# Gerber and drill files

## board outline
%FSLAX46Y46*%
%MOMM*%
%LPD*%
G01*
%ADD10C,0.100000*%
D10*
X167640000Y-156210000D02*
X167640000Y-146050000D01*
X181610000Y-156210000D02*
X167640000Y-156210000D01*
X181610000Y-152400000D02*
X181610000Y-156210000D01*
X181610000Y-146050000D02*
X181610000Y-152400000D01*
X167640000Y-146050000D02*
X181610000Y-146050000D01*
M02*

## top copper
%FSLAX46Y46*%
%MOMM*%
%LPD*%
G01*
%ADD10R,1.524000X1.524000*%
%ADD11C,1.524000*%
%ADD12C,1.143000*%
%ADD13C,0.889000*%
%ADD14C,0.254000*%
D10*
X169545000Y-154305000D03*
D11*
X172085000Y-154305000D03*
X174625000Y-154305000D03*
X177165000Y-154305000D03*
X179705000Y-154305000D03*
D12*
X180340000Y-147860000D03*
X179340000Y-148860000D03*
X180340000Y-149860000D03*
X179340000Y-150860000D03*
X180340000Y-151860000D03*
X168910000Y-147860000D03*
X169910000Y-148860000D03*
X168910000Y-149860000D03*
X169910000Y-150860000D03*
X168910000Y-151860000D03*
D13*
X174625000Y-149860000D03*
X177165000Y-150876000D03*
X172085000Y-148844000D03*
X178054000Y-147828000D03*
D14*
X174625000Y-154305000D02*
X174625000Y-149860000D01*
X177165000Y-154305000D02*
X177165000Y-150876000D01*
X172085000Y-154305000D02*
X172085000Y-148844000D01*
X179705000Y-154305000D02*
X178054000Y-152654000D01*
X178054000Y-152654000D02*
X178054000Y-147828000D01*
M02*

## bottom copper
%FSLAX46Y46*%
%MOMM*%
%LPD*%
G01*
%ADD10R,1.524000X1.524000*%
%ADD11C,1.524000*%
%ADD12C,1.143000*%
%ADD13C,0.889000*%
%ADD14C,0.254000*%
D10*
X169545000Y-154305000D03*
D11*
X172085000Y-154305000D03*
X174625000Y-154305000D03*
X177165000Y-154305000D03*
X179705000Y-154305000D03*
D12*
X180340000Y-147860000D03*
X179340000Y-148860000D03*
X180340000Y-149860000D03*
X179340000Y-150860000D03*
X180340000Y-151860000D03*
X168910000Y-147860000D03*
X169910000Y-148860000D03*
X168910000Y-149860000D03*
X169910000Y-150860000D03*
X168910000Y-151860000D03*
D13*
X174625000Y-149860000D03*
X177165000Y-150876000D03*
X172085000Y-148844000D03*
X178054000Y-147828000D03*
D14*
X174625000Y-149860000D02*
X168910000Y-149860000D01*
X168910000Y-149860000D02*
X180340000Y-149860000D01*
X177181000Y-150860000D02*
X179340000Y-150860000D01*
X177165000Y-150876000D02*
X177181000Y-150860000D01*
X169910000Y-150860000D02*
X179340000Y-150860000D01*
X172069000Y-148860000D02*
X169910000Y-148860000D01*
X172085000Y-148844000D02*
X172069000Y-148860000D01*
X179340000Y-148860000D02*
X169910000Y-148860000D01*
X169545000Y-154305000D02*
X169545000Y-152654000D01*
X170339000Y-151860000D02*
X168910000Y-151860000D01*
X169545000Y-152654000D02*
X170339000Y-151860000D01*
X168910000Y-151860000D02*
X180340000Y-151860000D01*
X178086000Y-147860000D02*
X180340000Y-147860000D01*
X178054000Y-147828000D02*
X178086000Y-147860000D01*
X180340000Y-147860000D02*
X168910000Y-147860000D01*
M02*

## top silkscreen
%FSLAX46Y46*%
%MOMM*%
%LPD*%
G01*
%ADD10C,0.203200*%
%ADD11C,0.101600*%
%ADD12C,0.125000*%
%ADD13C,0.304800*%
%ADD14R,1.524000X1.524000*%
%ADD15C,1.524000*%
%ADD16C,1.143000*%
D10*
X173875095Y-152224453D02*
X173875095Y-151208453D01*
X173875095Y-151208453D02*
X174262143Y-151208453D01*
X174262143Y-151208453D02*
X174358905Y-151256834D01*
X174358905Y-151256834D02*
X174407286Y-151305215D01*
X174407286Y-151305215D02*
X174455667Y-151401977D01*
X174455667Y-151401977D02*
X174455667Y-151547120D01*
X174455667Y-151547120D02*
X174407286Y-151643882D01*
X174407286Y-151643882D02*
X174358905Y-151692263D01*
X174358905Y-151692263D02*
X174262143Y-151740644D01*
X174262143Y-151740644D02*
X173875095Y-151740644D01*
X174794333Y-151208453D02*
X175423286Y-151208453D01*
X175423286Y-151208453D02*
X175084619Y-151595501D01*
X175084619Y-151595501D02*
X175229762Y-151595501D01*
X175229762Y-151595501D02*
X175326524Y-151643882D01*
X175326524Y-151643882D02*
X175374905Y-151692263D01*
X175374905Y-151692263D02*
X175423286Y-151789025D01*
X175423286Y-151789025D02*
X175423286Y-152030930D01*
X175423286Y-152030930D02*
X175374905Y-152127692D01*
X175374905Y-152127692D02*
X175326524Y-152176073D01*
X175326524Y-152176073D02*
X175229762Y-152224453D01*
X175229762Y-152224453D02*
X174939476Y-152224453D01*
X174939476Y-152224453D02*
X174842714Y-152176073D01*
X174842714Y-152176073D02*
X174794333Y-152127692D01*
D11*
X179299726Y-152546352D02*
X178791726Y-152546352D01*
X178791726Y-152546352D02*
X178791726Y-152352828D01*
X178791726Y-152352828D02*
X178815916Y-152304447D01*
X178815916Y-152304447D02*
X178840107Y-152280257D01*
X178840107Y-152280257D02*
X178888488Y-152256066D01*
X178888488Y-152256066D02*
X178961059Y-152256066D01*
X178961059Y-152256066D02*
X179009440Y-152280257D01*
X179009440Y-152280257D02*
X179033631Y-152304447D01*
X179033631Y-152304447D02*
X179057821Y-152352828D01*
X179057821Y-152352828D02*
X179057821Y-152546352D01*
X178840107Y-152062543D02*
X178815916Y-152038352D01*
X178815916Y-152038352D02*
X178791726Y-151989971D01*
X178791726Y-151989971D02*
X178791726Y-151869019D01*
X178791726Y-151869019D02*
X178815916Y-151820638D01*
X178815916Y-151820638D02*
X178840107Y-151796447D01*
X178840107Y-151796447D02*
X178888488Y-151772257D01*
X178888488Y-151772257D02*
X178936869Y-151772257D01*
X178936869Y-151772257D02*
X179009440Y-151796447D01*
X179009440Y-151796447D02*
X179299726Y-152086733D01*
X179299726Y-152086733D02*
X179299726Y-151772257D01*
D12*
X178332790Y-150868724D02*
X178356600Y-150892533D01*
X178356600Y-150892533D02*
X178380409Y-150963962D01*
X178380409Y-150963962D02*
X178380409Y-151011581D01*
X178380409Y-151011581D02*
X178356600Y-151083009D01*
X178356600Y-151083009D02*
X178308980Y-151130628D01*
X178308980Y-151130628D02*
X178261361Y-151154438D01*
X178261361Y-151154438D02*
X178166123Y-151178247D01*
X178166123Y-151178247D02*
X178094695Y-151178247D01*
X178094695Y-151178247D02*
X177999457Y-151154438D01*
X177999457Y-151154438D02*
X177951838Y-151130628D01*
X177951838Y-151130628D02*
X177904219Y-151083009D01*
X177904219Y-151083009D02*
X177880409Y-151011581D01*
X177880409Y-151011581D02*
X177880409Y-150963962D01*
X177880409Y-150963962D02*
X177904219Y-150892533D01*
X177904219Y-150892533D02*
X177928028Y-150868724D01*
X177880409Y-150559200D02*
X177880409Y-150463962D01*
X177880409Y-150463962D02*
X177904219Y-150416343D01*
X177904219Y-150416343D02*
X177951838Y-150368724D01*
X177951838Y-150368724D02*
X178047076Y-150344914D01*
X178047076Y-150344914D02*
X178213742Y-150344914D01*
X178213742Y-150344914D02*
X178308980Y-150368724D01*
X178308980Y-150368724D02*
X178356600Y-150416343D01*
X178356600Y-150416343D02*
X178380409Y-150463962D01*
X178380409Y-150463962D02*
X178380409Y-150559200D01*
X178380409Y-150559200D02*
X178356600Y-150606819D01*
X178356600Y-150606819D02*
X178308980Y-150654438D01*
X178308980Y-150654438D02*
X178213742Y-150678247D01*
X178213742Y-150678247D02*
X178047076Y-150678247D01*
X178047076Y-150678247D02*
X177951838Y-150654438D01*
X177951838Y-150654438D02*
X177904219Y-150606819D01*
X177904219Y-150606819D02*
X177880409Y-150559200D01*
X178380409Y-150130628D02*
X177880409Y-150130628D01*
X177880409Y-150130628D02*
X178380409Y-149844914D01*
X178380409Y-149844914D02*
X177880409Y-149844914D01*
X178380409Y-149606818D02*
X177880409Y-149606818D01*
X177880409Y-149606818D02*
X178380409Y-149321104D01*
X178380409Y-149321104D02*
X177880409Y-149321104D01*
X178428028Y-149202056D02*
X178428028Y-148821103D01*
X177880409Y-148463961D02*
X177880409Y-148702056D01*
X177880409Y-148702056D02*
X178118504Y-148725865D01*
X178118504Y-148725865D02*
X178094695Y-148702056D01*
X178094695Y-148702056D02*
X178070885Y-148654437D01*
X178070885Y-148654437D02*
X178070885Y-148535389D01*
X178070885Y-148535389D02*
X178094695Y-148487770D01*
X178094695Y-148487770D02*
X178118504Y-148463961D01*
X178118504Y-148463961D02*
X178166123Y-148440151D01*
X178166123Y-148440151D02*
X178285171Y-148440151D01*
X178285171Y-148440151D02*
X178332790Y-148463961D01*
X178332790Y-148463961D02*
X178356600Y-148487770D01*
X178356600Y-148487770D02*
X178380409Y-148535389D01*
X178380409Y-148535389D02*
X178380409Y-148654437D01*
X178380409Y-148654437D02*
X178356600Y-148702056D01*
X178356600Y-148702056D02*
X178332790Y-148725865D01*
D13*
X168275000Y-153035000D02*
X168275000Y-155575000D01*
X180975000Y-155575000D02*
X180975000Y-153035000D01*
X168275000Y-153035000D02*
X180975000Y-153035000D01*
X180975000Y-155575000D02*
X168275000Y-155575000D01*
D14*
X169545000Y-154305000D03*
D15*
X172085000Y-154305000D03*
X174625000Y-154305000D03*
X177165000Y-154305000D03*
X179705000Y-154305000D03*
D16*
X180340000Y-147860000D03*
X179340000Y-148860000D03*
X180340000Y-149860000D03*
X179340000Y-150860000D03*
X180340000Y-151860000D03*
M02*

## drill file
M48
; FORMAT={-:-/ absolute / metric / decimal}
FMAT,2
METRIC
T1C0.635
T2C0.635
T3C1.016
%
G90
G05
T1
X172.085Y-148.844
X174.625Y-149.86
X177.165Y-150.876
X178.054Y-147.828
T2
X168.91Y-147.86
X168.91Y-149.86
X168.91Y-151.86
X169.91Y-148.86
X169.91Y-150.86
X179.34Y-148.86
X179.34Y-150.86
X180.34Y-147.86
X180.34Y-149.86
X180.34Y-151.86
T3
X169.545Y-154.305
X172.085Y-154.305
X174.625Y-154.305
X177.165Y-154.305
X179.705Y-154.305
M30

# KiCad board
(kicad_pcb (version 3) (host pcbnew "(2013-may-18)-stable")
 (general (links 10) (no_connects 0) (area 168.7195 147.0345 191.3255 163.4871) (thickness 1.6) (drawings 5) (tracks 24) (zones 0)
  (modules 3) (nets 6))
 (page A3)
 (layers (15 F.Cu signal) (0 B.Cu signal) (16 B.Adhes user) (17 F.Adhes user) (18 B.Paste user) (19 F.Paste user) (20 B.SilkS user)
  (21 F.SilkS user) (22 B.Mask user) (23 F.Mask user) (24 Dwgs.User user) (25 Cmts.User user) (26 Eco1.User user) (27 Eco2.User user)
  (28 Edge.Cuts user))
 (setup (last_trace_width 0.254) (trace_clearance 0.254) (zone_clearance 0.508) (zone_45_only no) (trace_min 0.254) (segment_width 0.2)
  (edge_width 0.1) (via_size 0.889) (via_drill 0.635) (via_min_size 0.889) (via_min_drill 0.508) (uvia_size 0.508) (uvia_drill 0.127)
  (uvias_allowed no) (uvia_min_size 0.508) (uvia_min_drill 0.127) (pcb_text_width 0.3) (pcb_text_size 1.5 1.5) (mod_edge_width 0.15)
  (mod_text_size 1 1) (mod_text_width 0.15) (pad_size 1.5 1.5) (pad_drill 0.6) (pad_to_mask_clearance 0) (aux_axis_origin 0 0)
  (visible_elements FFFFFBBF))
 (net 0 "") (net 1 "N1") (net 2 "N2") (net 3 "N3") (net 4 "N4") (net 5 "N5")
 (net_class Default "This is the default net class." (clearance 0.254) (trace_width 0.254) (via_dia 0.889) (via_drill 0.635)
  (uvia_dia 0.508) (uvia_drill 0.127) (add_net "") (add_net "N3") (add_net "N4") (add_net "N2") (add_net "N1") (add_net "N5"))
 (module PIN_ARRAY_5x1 (layer F.Cu) (at 174.625 154.305)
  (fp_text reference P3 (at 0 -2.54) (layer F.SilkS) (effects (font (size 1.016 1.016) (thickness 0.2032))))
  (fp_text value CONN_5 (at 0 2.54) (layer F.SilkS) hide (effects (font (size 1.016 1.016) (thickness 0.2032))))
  (fp_line (start -6.35 -1.27) (end -6.35 1.27) (layer F.SilkS) (width 0.3048))
  (fp_line (start 6.35 1.27) (end 6.35 -1.27) (layer F.SilkS) (width 0.3048))
  (fp_line (start -6.35 -1.27) (end 6.35 -1.27) (layer F.SilkS) (width 0.3048))
  (fp_line (start 6.35 1.27) (end -6.35 1.27) (layer F.SilkS) (width 0.3048))
  (pad 1 thru_hole rect (at -5.08 0) (size 1.524 1.524) (drill 1.016) (layers *.Cu *.Mask F.SilkS) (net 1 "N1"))
  (pad 2 thru_hole circle (at -2.54 0) (size 1.524 1.524) (drill 1.016) (layers *.Cu *.Mask F.SilkS) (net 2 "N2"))
  (pad 3 thru_hole circle (at 0 0) (size 1.524 1.524) (drill 1.016) (layers *.Cu *.Mask F.SilkS) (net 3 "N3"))
  (pad 4 thru_hole circle (at 2.54 0) (size 1.524 1.524) (drill 1.016) (layers *.Cu *.Mask F.SilkS) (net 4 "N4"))
  (pad 5 thru_hole circle (at 5.08 0) (size 1.524 1.524) (drill 1.016) (layers *.Cu *.Mask F.SilkS) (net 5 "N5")))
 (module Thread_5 (layer F.Cu) (at 180.34 149.86 270)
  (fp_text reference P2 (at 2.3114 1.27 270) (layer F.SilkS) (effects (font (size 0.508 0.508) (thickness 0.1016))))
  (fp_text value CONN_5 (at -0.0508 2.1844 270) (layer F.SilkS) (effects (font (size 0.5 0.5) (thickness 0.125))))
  (pad 1 thru_hole circle (at -2 0 270) (size 1.143 1.143) (drill 0.635) (layers *.Cu *.Mask F.SilkS) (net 5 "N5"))
  (pad 2 thru_hole circle (at -1 1 270) (size 1.143 1.143) (drill 0.635) (layers *.Cu *.Mask F.SilkS) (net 2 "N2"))
  (pad 3 thru_hole circle (at 0 0 270) (size 1.143 1.143) (drill 0.635) (layers *.Cu *.Mask F.SilkS) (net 3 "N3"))
  (pad 4 thru_hole circle (at 1 1 270) (size 1.143 1.143) (drill 0.635) (layers *.Cu *.Mask F.SilkS) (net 4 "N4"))
  (pad 5 thru_hole circle (at 2 0 270) (size 1.143 1.143) (drill 0.635) (layers *.Cu *.Mask F.SilkS) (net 1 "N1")))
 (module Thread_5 (layer B.Cu) (at 168.91 149.86 270)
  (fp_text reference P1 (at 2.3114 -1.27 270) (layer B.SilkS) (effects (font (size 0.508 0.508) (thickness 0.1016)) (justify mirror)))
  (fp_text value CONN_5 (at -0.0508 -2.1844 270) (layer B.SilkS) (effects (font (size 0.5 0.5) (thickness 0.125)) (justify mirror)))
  (pad 1 thru_hole circle (at -2 0 270) (size 1.143 1.143) (drill 0.635) (layers *.Cu *.Mask B.SilkS) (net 5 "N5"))
  (pad 2 thru_hole circle (at -1 -1 270) (size 1.143 1.143) (drill 0.635) (layers *.Cu *.Mask B.SilkS) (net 2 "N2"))
  (pad 3 thru_hole circle (at 0 0 270) (size 1.143 1.143) (drill 0.635) (layers *.Cu *.Mask B.SilkS) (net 3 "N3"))
  (pad 4 thru_hole circle (at 1 -1 270) (size 1.143 1.143) (drill 0.635) (layers *.Cu *.Mask B.SilkS) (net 4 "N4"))
  (pad 5 thru_hole circle (at 2 0 270) (size 1.143 1.143) (drill 0.635) (layers *.Cu *.Mask B.SilkS) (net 1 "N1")))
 (gr_line (start 167.64 156.21) (end 167.64 146.05) (angle 90) (layer Edge.Cuts) (width 0.1))
 (gr_line (start 181.61 156.21) (end 167.64 156.21) (angle 90) (layer Edge.Cuts) (width 0.1))
 (gr_line (start 181.61 152.4) (end 181.61 156.21) (angle 90) (layer Edge.Cuts) (width 0.1))
 (gr_line (start 181.61 146.05) (end 181.61 152.4) (angle 90) (layer Edge.Cuts) (width 0.1))
 (gr_line (start 167.64 146.05) (end 181.61 146.05) (angle 90) (layer Edge.Cuts) (width 0.1))
 (segment (start 174.625 154.305) (end 174.625 149.86) (width 0.254) (layer F.Cu) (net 3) (status 400000))
 (segment (start 174.625 149.86) (end 168.91 149.86) (width 0.254) (layer B.Cu) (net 3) (status 800000))
 (via (at 174.625 149.86) (size 0.889) (layers F.Cu B.Cu) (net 3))
 (segment (start 168.91 149.86) (end 180.34 149.86) (width 0.254) (layer B.Cu) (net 3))
 (segment (start 177.165 154.305) (end 177.165 150.876) (width 0.254) (layer F.Cu) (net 4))
 (segment (start 177.181 150.86) (end 179.34 150.86) (width 0.254) (layer B.Cu) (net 4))
 (segment (start 177.165 150.876) (end 177.181 150.86) (width 0.254) (layer B.Cu) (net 4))
 (via (at 177.165 150.876) (size 0.889) (layers F.Cu B.Cu) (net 4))
 (segment (start 169.91 150.86) (end 179.34 150.86) (width 0.254) (layer B.Cu) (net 4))
 (segment (start 172.085 154.305) (end 172.085 148.844) (width 0.254) (layer F.Cu) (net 2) (status 400000))
 (segment (start 172.069 148.86) (end 169.91 148.86) (width 0.254) (layer B.Cu) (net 2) (status 800000))
 (segment (start 172.085 148.844) (end 172.069 148.86) (width 0.254) (layer B.Cu) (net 2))
 (via (at 172.085 148.844) (size 0.889) (layers F.Cu B.Cu) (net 2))
 (segment (start 179.34 148.86) (end 169.91 148.86) (width 0.254) (layer B.Cu) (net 2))
 (segment (start 169.545 154.305) (end 169.545 152.654) (width 0.254) (layer B.Cu) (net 1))
 (segment (start 170.339 151.86) (end 168.91 151.86) (width 0.254) (layer B.Cu) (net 1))
 (segment (start 169.545 152.654) (end 170.339 151.86) (width 0.254) (layer B.Cu) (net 1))
 (segment (start 168.91 151.86) (end 180.34 151.86) (width 0.254) (layer B.Cu) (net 1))
 (segment (start 179.705 154.305) (end 178.054 152.654) (width 0.254) (layer F.Cu) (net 5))
 (segment (start 178.086 147.86) (end 180.34 147.86) (width 0.254) (layer B.Cu) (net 5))
 (segment (start 178.054 147.828) (end 178.086 147.86) (width 0.254) (layer B.Cu) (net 5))
 (via (at 178.054 147.828) (size 0.889) (layers F.Cu B.Cu) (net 5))
 (segment (start 178.054 152.654) (end 178.054 147.828) (width 0.254) (layer F.Cu) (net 5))
 (segment (start 180.34 147.86) (end 168.91 147.86) (width 0.254) (layer B.Cu) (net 5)))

